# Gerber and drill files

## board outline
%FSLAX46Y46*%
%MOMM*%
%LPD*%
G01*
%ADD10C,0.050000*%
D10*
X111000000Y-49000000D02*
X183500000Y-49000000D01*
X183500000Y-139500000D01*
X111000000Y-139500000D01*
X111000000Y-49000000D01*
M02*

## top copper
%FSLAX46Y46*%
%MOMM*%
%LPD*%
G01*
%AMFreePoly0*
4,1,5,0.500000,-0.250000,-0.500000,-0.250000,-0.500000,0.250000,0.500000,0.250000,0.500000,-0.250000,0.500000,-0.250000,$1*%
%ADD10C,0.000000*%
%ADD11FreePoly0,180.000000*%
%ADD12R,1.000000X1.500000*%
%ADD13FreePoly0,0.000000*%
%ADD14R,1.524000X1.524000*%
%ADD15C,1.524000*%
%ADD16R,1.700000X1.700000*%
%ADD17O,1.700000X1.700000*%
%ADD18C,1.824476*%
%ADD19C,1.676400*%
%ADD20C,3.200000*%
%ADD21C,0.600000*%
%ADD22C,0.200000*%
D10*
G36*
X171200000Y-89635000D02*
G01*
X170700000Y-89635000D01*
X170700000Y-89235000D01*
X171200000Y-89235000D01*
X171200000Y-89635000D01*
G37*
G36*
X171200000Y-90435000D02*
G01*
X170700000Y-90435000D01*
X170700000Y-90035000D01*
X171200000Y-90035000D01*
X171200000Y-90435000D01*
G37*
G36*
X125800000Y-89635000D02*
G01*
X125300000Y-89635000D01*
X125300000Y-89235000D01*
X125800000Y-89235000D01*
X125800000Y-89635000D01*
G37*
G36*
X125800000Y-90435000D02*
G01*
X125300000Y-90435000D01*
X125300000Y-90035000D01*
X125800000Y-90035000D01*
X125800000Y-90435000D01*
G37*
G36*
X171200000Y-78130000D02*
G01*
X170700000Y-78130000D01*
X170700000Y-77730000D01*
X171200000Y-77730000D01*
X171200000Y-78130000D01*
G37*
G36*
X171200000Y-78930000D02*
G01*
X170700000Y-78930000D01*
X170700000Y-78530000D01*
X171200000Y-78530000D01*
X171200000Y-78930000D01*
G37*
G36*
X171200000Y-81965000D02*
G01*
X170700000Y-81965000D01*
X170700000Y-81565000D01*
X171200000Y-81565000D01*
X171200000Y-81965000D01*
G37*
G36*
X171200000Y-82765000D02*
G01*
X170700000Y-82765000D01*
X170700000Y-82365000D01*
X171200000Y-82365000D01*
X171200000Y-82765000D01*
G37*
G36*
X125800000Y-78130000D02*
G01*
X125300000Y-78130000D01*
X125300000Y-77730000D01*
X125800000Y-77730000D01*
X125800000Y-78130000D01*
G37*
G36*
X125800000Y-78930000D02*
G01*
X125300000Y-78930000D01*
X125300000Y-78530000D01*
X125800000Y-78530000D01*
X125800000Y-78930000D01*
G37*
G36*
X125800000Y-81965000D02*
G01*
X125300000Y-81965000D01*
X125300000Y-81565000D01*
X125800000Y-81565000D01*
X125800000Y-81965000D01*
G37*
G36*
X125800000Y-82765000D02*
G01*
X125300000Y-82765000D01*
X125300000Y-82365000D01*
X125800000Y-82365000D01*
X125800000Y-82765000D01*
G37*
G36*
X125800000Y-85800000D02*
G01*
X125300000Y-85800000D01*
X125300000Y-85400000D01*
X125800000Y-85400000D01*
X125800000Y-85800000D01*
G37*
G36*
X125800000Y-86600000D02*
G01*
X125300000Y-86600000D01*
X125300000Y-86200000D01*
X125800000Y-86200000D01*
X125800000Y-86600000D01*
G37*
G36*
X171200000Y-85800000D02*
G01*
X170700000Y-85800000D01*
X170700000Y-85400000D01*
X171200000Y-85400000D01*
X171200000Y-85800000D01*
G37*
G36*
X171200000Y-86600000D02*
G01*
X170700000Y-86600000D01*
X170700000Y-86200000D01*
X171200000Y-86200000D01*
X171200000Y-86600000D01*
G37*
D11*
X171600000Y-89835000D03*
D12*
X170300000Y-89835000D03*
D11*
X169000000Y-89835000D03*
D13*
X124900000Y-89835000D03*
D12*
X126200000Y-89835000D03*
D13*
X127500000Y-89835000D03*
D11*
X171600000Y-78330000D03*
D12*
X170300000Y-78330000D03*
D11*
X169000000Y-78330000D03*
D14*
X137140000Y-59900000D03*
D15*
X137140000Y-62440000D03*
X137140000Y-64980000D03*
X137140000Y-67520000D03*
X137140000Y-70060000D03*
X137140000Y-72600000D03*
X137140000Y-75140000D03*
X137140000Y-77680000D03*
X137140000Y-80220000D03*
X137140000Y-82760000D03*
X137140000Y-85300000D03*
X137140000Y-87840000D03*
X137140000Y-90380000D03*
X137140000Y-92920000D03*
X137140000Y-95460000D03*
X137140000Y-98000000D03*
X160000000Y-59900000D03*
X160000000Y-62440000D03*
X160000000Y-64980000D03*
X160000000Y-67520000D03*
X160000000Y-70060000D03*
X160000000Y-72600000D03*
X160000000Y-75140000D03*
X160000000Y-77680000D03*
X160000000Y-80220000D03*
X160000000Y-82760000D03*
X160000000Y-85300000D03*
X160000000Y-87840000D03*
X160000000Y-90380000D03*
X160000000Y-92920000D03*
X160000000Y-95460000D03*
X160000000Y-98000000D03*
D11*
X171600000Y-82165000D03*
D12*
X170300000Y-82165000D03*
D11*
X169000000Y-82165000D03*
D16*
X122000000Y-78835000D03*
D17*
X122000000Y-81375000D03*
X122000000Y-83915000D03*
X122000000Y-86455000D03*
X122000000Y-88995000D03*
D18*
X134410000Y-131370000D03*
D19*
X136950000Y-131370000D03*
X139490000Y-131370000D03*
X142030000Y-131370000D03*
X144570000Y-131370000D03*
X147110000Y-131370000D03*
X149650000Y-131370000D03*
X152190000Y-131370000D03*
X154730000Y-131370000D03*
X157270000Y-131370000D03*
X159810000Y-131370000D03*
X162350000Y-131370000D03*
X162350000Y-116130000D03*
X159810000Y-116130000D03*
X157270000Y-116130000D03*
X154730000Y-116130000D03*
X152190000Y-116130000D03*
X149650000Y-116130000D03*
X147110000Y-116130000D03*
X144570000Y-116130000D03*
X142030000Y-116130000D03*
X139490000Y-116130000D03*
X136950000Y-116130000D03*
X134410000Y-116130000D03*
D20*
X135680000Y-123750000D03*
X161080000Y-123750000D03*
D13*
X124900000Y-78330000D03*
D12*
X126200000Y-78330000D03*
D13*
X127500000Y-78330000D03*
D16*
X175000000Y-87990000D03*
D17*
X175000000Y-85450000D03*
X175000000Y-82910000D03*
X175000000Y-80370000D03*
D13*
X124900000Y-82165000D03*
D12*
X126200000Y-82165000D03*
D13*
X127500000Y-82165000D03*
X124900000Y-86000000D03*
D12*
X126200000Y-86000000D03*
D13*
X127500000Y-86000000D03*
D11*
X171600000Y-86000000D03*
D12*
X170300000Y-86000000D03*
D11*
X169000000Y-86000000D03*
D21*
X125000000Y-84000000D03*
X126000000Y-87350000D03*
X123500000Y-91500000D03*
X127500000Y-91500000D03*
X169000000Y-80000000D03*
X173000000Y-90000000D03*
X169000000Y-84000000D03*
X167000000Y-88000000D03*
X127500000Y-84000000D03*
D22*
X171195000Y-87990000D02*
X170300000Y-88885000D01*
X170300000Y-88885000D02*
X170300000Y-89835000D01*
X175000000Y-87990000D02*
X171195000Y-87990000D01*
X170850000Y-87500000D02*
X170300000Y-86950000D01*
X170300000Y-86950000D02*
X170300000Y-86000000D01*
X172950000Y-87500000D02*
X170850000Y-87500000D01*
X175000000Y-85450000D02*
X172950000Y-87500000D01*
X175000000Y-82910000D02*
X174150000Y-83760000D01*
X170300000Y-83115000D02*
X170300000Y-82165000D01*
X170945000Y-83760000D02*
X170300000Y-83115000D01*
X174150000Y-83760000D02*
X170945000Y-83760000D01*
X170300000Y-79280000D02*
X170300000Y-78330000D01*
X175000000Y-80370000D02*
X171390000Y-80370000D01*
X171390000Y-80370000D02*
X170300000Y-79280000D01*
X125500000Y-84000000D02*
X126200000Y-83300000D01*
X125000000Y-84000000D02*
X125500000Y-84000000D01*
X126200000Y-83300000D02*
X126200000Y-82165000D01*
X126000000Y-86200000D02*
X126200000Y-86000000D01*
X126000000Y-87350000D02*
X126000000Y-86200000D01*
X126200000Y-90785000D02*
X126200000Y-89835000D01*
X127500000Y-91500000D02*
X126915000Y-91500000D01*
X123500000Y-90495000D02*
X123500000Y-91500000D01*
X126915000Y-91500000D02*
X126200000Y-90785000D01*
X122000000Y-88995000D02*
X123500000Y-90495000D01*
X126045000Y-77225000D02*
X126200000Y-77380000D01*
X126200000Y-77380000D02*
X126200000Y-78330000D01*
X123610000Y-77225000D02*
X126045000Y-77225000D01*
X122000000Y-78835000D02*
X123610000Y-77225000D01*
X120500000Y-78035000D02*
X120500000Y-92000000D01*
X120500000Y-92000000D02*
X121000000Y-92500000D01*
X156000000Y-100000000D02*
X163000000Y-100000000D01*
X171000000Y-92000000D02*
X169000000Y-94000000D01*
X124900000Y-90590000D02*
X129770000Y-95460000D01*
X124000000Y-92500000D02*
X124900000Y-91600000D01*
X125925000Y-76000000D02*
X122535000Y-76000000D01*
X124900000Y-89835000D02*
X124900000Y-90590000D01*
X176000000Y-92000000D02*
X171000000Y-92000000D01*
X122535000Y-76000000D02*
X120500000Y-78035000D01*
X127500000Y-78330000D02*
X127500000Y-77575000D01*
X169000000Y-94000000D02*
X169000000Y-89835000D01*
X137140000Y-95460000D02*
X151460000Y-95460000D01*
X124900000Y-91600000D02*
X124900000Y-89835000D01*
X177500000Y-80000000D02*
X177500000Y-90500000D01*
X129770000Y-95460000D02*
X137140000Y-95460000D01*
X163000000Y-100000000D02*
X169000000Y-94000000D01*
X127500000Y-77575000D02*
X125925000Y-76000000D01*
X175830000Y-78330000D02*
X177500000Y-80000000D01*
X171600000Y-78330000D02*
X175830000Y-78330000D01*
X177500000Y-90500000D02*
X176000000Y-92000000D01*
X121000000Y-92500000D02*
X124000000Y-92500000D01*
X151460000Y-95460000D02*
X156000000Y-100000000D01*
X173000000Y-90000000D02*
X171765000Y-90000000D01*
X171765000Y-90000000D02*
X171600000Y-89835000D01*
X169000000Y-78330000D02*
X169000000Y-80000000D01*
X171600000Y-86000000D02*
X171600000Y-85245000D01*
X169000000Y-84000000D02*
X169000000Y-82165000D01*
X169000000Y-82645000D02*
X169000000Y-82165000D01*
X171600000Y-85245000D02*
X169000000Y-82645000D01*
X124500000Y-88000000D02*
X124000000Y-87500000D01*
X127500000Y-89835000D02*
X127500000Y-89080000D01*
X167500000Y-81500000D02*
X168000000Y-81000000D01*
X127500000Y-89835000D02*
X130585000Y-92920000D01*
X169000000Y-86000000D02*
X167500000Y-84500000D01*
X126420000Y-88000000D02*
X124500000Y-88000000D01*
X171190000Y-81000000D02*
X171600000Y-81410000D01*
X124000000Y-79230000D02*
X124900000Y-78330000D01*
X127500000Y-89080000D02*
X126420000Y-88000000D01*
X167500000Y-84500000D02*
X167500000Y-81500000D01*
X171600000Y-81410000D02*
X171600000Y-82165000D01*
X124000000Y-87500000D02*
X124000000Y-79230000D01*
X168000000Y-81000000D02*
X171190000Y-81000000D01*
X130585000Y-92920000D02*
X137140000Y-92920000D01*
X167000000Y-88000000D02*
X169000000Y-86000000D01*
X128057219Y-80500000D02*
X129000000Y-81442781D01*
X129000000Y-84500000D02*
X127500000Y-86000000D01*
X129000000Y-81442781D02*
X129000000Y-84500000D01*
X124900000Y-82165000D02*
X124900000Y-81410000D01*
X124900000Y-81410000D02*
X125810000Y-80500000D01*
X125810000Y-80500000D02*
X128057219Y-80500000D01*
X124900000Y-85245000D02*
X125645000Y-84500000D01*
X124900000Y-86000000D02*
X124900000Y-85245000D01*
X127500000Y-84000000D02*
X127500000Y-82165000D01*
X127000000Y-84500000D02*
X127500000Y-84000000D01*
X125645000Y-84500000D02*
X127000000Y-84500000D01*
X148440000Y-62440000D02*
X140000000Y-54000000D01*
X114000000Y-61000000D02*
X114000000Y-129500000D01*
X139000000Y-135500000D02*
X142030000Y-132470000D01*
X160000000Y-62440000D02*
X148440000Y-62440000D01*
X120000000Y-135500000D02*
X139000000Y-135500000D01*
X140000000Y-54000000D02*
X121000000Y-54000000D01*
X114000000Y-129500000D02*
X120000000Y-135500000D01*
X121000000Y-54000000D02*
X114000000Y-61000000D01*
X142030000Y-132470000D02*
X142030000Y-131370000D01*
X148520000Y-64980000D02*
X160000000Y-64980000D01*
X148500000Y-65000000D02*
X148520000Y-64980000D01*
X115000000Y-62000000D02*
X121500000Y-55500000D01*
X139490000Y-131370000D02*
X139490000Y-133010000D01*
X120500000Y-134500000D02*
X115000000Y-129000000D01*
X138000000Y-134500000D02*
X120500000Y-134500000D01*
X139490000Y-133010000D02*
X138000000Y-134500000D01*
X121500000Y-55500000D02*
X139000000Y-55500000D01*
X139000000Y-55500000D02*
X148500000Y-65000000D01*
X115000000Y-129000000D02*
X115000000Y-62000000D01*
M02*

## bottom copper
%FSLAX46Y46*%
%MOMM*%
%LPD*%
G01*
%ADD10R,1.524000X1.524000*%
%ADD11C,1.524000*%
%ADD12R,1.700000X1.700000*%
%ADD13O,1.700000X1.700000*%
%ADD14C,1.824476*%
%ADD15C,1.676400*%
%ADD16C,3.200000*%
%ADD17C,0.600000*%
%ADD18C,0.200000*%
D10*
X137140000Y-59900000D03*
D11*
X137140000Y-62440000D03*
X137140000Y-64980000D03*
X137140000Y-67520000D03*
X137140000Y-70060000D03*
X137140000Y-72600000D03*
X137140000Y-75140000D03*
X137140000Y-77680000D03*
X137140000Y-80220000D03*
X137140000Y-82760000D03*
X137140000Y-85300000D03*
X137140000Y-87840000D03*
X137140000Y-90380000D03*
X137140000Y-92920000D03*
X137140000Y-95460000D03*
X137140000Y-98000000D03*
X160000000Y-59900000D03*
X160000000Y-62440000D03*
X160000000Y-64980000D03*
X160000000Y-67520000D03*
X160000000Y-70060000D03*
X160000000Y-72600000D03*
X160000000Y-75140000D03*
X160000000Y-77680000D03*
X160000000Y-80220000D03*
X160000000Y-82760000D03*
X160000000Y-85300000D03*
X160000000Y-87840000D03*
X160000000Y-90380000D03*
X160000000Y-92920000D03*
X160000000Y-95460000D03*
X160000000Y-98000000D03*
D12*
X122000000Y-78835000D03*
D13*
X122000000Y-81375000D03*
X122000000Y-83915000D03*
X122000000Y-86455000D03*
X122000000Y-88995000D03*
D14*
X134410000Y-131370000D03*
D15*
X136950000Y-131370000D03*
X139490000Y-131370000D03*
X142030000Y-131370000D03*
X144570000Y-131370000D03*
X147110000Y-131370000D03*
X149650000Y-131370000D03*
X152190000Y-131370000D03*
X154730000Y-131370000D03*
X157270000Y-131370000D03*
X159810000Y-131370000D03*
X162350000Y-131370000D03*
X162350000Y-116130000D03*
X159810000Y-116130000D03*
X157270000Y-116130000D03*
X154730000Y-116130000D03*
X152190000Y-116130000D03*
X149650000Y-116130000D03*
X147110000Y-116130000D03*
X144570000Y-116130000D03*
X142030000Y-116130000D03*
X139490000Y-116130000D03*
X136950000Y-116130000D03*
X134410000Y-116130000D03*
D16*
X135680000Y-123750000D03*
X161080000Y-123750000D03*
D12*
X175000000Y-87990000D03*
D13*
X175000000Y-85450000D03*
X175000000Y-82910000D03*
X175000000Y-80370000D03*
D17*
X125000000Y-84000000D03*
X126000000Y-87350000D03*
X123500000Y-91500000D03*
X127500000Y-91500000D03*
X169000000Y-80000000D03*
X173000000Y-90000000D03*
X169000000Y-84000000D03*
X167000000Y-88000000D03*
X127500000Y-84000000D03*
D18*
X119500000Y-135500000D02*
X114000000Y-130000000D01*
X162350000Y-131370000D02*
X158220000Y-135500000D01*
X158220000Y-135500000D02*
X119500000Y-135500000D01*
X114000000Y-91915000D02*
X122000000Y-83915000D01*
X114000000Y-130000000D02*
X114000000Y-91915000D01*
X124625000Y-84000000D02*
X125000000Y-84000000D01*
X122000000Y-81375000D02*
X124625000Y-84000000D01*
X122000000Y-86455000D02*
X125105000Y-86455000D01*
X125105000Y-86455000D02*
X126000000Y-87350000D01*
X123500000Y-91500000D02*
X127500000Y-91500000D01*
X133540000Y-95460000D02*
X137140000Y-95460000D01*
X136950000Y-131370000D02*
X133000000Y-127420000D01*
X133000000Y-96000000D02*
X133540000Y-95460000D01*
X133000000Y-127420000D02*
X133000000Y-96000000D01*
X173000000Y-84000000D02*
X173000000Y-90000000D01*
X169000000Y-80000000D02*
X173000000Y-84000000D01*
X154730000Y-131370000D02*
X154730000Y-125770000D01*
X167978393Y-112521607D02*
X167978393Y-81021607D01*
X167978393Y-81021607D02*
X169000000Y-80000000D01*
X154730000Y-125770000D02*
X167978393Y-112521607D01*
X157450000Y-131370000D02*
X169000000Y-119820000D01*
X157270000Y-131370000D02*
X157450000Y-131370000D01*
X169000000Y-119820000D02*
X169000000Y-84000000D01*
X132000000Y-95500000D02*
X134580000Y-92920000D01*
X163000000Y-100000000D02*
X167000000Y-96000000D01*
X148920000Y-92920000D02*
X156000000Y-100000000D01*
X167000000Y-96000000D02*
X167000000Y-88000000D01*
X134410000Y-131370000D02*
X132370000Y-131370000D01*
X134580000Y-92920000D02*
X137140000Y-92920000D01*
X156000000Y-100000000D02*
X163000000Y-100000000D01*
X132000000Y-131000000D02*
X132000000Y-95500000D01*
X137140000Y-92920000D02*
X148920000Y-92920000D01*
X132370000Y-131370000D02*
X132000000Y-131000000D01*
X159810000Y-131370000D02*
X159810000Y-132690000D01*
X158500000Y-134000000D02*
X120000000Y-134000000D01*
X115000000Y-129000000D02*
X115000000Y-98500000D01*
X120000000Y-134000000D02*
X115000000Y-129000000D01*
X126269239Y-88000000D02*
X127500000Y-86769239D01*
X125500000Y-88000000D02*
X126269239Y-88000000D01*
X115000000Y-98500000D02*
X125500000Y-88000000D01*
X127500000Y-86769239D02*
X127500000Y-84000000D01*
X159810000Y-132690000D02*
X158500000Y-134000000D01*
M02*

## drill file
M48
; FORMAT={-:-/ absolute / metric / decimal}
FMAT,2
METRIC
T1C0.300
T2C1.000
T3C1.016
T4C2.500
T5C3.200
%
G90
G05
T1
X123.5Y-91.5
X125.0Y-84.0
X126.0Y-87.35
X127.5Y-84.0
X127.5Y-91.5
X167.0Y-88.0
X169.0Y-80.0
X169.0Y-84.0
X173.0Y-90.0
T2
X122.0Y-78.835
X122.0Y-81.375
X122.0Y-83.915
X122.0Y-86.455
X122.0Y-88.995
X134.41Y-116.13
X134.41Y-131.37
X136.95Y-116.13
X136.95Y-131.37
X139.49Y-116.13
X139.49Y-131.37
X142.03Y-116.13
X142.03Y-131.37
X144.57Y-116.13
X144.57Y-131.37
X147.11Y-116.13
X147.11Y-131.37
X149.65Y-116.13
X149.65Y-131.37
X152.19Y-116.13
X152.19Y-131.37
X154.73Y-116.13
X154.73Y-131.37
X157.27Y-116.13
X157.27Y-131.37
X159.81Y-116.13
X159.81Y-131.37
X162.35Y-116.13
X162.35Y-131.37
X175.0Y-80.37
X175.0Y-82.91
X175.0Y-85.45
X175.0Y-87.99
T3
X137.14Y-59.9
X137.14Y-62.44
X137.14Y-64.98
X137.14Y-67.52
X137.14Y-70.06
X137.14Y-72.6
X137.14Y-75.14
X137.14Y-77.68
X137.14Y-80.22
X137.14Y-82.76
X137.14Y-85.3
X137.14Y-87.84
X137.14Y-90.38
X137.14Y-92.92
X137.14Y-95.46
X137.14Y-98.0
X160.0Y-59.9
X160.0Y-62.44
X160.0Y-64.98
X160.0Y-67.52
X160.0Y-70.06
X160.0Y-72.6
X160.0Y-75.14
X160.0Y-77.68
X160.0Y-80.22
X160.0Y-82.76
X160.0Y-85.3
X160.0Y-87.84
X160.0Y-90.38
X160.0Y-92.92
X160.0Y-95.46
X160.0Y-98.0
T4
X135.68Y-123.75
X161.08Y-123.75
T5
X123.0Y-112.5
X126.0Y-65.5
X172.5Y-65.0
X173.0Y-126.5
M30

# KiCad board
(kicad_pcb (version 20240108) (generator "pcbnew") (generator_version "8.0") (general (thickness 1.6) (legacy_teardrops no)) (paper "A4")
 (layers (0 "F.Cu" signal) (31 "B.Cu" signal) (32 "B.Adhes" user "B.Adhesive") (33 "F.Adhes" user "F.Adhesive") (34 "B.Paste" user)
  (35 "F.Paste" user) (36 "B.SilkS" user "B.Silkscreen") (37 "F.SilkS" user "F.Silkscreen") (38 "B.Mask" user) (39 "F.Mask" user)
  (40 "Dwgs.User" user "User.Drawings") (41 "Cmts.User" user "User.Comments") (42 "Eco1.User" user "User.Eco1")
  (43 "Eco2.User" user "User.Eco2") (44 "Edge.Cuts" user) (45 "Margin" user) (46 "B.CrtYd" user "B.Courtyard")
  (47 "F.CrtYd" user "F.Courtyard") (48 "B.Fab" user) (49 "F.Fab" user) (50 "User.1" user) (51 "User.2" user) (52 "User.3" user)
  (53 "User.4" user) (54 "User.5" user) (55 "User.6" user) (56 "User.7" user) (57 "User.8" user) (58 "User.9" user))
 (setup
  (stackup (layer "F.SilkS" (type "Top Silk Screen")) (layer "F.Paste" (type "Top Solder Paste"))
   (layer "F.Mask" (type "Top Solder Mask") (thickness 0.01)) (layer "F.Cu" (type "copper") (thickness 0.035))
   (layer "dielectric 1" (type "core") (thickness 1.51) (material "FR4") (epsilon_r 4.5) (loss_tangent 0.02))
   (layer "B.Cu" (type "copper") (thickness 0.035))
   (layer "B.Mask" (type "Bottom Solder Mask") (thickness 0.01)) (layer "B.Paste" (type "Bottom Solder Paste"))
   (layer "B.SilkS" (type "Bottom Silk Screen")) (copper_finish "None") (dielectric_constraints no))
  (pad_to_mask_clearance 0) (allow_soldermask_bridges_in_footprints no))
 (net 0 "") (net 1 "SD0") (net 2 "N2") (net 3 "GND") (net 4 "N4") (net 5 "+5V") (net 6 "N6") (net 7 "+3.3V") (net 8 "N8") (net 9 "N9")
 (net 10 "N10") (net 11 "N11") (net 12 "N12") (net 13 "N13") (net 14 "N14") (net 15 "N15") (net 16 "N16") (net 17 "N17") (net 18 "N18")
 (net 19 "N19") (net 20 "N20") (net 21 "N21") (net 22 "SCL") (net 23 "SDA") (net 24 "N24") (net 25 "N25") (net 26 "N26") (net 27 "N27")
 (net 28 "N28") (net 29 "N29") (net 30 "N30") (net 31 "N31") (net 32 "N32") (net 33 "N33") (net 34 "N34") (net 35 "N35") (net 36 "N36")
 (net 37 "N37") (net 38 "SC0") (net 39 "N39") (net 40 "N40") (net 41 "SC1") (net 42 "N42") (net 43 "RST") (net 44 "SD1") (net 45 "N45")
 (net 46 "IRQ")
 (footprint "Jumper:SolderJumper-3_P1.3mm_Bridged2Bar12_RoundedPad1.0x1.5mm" (layer "F.Cu") (at 170.3 89.835 180)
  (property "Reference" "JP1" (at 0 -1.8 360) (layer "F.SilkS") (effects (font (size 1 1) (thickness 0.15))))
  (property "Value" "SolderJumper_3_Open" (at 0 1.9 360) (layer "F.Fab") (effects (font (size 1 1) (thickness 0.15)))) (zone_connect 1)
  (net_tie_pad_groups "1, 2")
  (fp_poly (pts (xy -0.9 0.2) (xy -0.4 0.2) (xy -0.4 0.6) (xy -0.9 0.6)) (stroke (width 0) (type solid)) (fill solid) (layer "F.Cu"))
  (fp_poly (pts (xy -0.9 -0.6) (xy -0.4 -0.6) (xy -0.4 -0.2) (xy -0.9 -0.2)) (stroke (width 0) (type solid)) (fill solid) (layer "F.Cu"))
  (pad "1" smd custom (at -1.3 0 180) (size 1 0.5) (layers "F.Cu" "F.Mask") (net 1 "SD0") (zone_connect 2) (thermal_bridge_angle 45)
   (options (clearance outline) (anchor rect)) (primitives))
  (pad "2" smd rect (at 0 0 180) (size 1 1.5) (layers "F.Cu" "F.Mask") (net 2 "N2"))
  (pad "3" smd custom (at 1.3 0 180) (size 1 0.5) (layers "F.Cu" "F.Mask") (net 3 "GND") (zone_connect 2) (thermal_bridge_angle 45)
   (options (clearance outline) (anchor rect)) (primitives)))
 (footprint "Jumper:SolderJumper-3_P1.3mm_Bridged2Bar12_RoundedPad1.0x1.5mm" (layer "F.Cu") (at 126.2 89.835)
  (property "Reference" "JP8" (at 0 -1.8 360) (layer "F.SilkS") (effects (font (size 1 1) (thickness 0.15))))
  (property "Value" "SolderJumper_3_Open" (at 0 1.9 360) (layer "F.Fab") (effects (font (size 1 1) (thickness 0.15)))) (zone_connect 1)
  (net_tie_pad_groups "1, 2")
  (fp_poly (pts (xy -0.9 -0.6) (xy -0.4 -0.6) (xy -0.4 -0.2) (xy -0.9 -0.2)) (stroke (width 0) (type solid)) (fill solid) (layer "F.Cu"))
  (fp_poly (pts (xy -0.9 0.2) (xy -0.4 0.2) (xy -0.4 0.6) (xy -0.9 0.6)) (stroke (width 0) (type solid)) (fill solid) (layer "F.Cu"))
  (pad "1" smd custom (at -1.3 0) (size 1 0.5) (layers "F.Cu" "F.Mask") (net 3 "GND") (zone_connect 2) (thermal_bridge_angle 45)
   (options (clearance outline) (anchor rect)) (primitives))
  (pad "2" smd rect (at 0 0) (size 1 1.5) (layers "F.Cu" "F.Mask") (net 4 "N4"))
  (pad "3" smd custom (at 1.3 0) (size 1 0.5) (layers "F.Cu" "F.Mask") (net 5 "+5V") (zone_connect 2) (thermal_bridge_angle 45)
   (options (clearance outline) (anchor rect)) (primitives)))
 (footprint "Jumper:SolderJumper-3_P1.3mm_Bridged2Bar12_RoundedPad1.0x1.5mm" (layer "F.Cu") (at 170.3 78.33 180)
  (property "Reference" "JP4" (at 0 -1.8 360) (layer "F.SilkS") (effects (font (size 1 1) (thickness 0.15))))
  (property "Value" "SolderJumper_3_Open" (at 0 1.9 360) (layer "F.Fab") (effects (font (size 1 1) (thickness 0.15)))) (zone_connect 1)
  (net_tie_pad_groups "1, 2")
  (fp_poly (pts (xy -0.9 0.2) (xy -0.4 0.2) (xy -0.4 0.6) (xy -0.9 0.6)) (stroke (width 0) (type solid)) (fill solid) (layer "F.Cu"))
  (fp_poly (pts (xy -0.9 -0.6) (xy -0.4 -0.6) (xy -0.4 -0.2) (xy -0.9 -0.2)) (stroke (width 0) (type solid)) (fill solid) (layer "F.Cu"))
  (pad "1" smd custom (at -1.3 0 180) (size 1 0.5) (layers "F.Cu" "F.Mask") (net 3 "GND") (zone_connect 2) (thermal_bridge_angle 45)
   (options (clearance outline) (anchor rect)) (primitives))
  (pad "2" smd rect (at 0 0 180) (size 1 1.5) (layers "F.Cu" "F.Mask") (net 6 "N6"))
  (pad "3" smd custom (at 1.3 0 180) (size 1 0.5) (layers "F.Cu" "F.Mask") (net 1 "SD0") (zone_connect 2) (thermal_bridge_angle 45)
   (options (clearance outline) (anchor rect)) (primitives)))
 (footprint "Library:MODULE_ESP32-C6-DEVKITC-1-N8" (layer "F.Cu") (at 148.57 84.225)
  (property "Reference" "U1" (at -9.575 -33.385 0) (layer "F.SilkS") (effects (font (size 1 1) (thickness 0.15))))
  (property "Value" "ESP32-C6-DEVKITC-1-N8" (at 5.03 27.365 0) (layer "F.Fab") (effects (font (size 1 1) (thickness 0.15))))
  (pad "J1_1" thru_hole rect (at -11.43 -24.325) (size 1.524 1.524) (drill 1.016) (layers "*.Cu" "*.Mask") (remove_unused_layers no)
   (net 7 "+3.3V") (solder_mask_margin 0.102))
  (pad "J1_2" thru_hole circle (at -11.43 -21.785) (size 1.524 1.524) (drill 1.016) (layers "*.Cu" "*.Mask") (remove_unused_layers no)
   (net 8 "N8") (solder_mask_margin 0.102))
  (pad "J1_3" thru_hole circle (at -11.43 -19.245) (size 1.524 1.524) (drill 1.016) (layers "*.Cu" "*.Mask") (remove_unused_layers no)
   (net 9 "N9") (solder_mask_margin 0.102))
  (pad "J1_4" thru_hole circle (at -11.43 -16.705) (size 1.524 1.524) (drill 1.016) (layers "*.Cu" "*.Mask") (remove_unused_layers no)
   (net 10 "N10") (solder_mask_margin 0.102))
  (pad "J1_5" thru_hole circle (at -11.43 -14.165) (size 1.524 1.524) (drill 1.016) (layers "*.Cu" "*.Mask") (remove_unused_layers no)
   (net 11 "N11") (solder_mask_margin 0.102))
  (pad "J1_6" thru_hole circle (at -11.43 -11.625) (size 1.524 1.524) (drill 1.016) (layers "*.Cu" "*.Mask") (remove_unused_layers no)
   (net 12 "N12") (solder_mask_margin 0.102))
  (pad "J1_7" thru_hole circle (at -11.43 -9.085) (size 1.524 1.524) (drill 1.016) (layers "*.Cu" "*.Mask") (remove_unused_layers no)
   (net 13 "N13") (solder_mask_margin 0.102))
  (pad "J1_8" thru_hole circle (at -11.43 -6.545) (size 1.524 1.524) (drill 1.016) (layers "*.Cu" "*.Mask") (remove_unused_layers no)
   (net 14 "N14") (solder_mask_margin 0.102))
  (pad "J1_9" thru_hole circle (at -11.43 -4.005) (size 1.524 1.524) (drill 1.016) (layers "*.Cu" "*.Mask") (remove_unused_layers no)
   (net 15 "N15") (solder_mask_margin 0.102))
  (pad "J1_10" thru_hole circle (at -11.43 -1.465) (size 1.524 1.524) (drill 1.016) (layers "*.Cu" "*.Mask") (remove_unused_layers no)
   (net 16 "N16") (solder_mask_margin 0.102))
  (pad "J1_11" thru_hole circle (at -11.43 1.075) (size 1.524 1.524) (drill 1.016) (layers "*.Cu" "*.Mask") (remove_unused_layers no)
   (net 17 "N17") (solder_mask_margin 0.102))
  (pad "J1_12" thru_hole circle (at -11.43 3.615) (size 1.524 1.524) (drill 1.016) (layers "*.Cu" "*.Mask") (remove_unused_layers no)
   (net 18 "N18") (solder_mask_margin 0.102))
  (pad "J1_13" thru_hole circle (at -11.43 6.155) (size 1.524 1.524) (drill 1.016) (layers "*.Cu" "*.Mask") (remove_unused_layers no)
   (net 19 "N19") (solder_mask_margin 0.102))
  (pad "J1_14" thru_hole circle (at -11.43 8.695) (size 1.524 1.524) (drill 1.016) (layers "*.Cu" "*.Mask") (remove_unused_layers no)
   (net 5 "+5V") (solder_mask_margin 0.102))
  (pad "J1_15" thru_hole circle (at -11.43 11.235) (size 1.524 1.524) (drill 1.016) (layers "*.Cu" "*.Mask") (remove_unused_layers no)
   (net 3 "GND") (solder_mask_margin 0.102))
  (pad "J1_16" thru_hole circle (at -11.43 13.775) (size 1.524 1.524) (drill 1.016) (layers "*.Cu" "*.Mask") (remove_unused_layers no)
   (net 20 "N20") (solder_mask_margin 0.102))
  (pad "J3_1" thru_hole circle (at 11.43 -24.325) (size 1.524 1.524) (drill 1.016) (layers "*.Cu" "*.Mask") (remove_unused_layers no)
   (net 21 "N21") (solder_mask_margin 0.102))
  (pad "J3_2" thru_hole circle (at 11.43 -21.785) (size 1.524 1.524) (drill 1.016) (layers "*.Cu" "*.Mask") (remove_unused_layers no)
   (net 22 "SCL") (solder_mask_margin 0.102))
  (pad "J3_3" thru_hole circle (at 11.43 -19.245) (size 1.524 1.524) (drill 1.016) (layers "*.Cu" "*.Mask") (remove_unused_layers no)
   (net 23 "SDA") (solder_mask_margin 0.102))
  (pad "J3_4" thru_hole circle (at 11.43 -16.705) (size 1.524 1.524) (drill 1.016) (layers "*.Cu" "*.Mask") (remove_unused_layers no)
   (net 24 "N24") (solder_mask_margin 0.102))
  (pad "J3_5" thru_hole circle (at 11.43 -14.165) (size 1.524 1.524) (drill 1.016) (layers "*.Cu" "*.Mask") (remove_unused_layers no)
   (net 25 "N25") (solder_mask_margin 0.102))
  (pad "J3_6" thru_hole circle (at 11.43 -11.625) (size 1.524 1.524) (drill 1.016) (layers "*.Cu" "*.Mask") (remove_unused_layers no)
   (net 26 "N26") (solder_mask_margin 0.102))
  (pad "J3_7" thru_hole circle (at 11.43 -9.085) (size 1.524 1.524) (drill 1.016) (layers "*.Cu" "*.Mask") (remove_unused_layers no)
   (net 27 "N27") (solder_mask_margin 0.102))
  (pad "J3_8" thru_hole circle (at 11.43 -6.545) (size 1.524 1.524) (drill 1.016) (layers "*.Cu" "*.Mask") (remove_unused_layers no)
   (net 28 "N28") (solder_mask_margin 0.102))
  (pad "J3_9" thru_hole circle (at 11.43 -4.005) (size 1.524 1.524) (drill 1.016) (layers "*.Cu" "*.Mask") (remove_unused_layers no)
   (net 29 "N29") (solder_mask_margin 0.102))
  (pad "J3_10" thru_hole circle (at 11.43 -1.465) (size 1.524 1.524) (drill 1.016) (layers "*.Cu" "*.Mask") (remove_unused_layers no)
   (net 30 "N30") (solder_mask_margin 0.102))
  (pad "J3_11" thru_hole circle (at 11.43 1.075) (size 1.524 1.524) (drill 1.016) (layers "*.Cu" "*.Mask") (remove_unused_layers no)
   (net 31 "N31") (solder_mask_margin 0.102))
  (pad "J3_12" thru_hole circle (at 11.43 3.615) (size 1.524 1.524) (drill 1.016) (layers "*.Cu" "*.Mask") (remove_unused_layers no)
   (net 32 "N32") (solder_mask_margin 0.102))
  (pad "J3_13" thru_hole circle (at 11.43 6.155) (size 1.524 1.524) (drill 1.016) (layers "*.Cu" "*.Mask") (remove_unused_layers no)
   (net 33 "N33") (solder_mask_margin 0.102))
  (pad "J3_14" thru_hole circle (at 11.43 8.695) (size 1.524 1.524) (drill 1.016) (layers "*.Cu" "*.Mask") (remove_unused_layers no)
   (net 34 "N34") (solder_mask_margin 0.102))
  (pad "J3_15" thru_hole circle (at 11.43 11.235) (size 1.524 1.524) (drill 1.016) (layers "*.Cu" "*.Mask") (remove_unused_layers no)
   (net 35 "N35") (solder_mask_margin 0.102))
  (pad "J3_16" thru_hole circle (at 11.43 13.775) (size 1.524 1.524) (drill 1.016) (layers "*.Cu" "*.Mask") (remove_unused_layers no)
   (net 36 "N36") (solder_mask_margin 0.102)))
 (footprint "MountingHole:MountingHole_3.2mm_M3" (layer "F.Cu") (at 173 126.5)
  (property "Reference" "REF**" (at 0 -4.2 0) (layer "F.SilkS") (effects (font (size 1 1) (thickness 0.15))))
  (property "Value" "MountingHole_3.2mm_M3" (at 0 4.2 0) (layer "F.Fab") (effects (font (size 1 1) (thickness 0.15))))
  (pad "" np_thru_hole circle (at 0 0) (size 3.2 3.2) (drill 3.2) (layers "F&B.Cu" "*.Mask")))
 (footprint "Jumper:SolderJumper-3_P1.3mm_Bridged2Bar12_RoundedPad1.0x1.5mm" (layer "F.Cu") (at 170.3 82.165 180)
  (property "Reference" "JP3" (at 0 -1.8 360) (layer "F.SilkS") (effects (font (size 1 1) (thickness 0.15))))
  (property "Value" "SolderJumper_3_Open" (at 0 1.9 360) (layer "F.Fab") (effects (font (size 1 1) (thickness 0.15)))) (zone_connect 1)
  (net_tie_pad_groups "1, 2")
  (fp_poly (pts (xy -0.9 0.2) (xy -0.4 0.2) (xy -0.4 0.6) (xy -0.9 0.6)) (stroke (width 0) (type solid)) (fill solid) (layer "F.Cu"))
  (fp_poly (pts (xy -0.9 -0.6) (xy -0.4 -0.6) (xy -0.4 -0.2) (xy -0.9 -0.2)) (stroke (width 0) (type solid)) (fill solid) (layer "F.Cu"))
  (pad "1" smd custom (at -1.3 0 180) (size 1 0.5) (layers "F.Cu" "F.Mask") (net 5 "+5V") (zone_connect 2) (thermal_bridge_angle 45)
   (options (clearance outline) (anchor rect)) (primitives))
  (pad "2" smd rect (at 0 0 180) (size 1 1.5) (layers "F.Cu" "F.Mask") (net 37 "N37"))
  (pad "3" smd custom (at 1.3 0 180) (size 1 0.5) (layers "F.Cu" "F.Mask") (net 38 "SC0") (zone_connect 2) (thermal_bridge_angle 45)
   (options (clearance outline) (anchor rect)) (primitives)))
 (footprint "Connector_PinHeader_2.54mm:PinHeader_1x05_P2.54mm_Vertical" (layer "F.Cu") (at 122 78.835)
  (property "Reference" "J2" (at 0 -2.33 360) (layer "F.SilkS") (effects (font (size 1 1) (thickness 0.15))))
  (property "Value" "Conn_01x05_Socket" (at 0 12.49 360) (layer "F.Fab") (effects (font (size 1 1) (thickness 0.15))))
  (pad "1" thru_hole rect (at 0 0) (size 1.7 1.7) (drill 1) (layers "*.Cu" "*.Mask") (remove_unused_layers no) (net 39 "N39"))
  (pad "2" thru_hole oval (at 0 2.54) (size 1.7 1.7) (drill 1) (layers "*.Cu" "*.Mask") (remove_unused_layers no) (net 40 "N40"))
  (pad "3" thru_hole oval (at 0 5.08) (size 1.7 1.7) (drill 1) (layers "*.Cu" "*.Mask") (remove_unused_layers no) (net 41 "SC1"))
  (pad "4" thru_hole oval (at 0 7.62) (size 1.7 1.7) (drill 1) (layers "*.Cu" "*.Mask") (remove_unused_layers no) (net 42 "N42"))
  (pad "5" thru_hole oval (at 0 10.16) (size 1.7 1.7) (drill 1) (layers "*.Cu" "*.Mask") (remove_unused_layers no) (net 4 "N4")))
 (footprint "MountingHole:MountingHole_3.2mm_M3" (layer "F.Cu") (at 123 112.5)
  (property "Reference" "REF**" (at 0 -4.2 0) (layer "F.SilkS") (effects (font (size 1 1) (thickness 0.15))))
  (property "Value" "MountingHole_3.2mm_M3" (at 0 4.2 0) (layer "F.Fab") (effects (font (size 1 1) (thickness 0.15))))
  (pad "" np_thru_hole circle (at 0 0) (size 3.2 3.2) (drill 3.2) (layers "F&B.Cu" "*.Mask")))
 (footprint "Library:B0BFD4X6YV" (layer "F.Cu") (at 129.27 123.13 90)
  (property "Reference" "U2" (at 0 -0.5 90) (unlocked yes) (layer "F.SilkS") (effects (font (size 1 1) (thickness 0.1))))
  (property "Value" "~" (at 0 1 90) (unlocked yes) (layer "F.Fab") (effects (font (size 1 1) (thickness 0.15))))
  (pad "1" thru_hole circle (at -8.24 5.14 90) (size 1.824476 1.824476) (drill 1) (layers "*.Cu" "*.Mask") (remove_unused_layers no)
   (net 5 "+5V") (solder_mask_margin 0.0508) (thermal_bridge_angle 0))
  (pad "2" thru_hole circle (at -8.24 7.68 90) (size 1.6764 1.6764) (drill 1) (layers "*.Cu" "*.Mask") (remove_unused_layers no)
   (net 3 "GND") (solder_mask_margin 0.0508) (thermal_bridge_angle 0))
  (pad "3" thru_hole circle (at -8.24 10.22 90) (size 1.6764 1.6764) (drill 1) (layers "*.Cu" "*.Mask") (remove_unused_layers no)
   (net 23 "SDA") (solder_mask_margin 0.0508) (thermal_bridge_angle 0))
  (pad "4" thru_hole circle (at -8.24 12.76 90) (size 1.6764 1.6764) (drill 1) (layers "*.Cu" "*.Mask") (remove_unused_layers no)
   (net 22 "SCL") (solder_mask_margin 0.0508) (thermal_bridge_angle 0))
  (pad "5" thru_hole circle (at -8.24 15.3 90) (size 1.6764 1.6764) (drill 1) (layers "*.Cu" "*.Mask") (remove_unused_layers no)
   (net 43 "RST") (solder_mask_margin 0.0508) (thermal_bridge_angle 0))
  (pad "6" thru_hole circle (at -8.24 17.84 90) (size 1.6764 1.6764) (drill 1) (layers "*.Cu" "*.Mask") (remove_unused_layers no)
   (solder_mask_margin 0.0508) (thermal_bridge_angle 0))
  (pad "7" thru_hole circle (at -8.24 20.38 90) (size 1.6764 1.6764) (drill 1) (layers "*.Cu" "*.Mask") (remove_unused_layers no)
   (solder_mask_margin 0.0508) (thermal_bridge_angle 0))
  (pad "8" thru_hole circle (at -8.24 22.92 90) (size 1.6764 1.6764) (drill 1) (layers "*.Cu" "*.Mask") (remove_unused_layers no)
   (solder_mask_margin 0.0508) (thermal_bridge_angle 0))
  (pad "9" thru_hole circle (at -8.24 25.46 90) (size 1.6764 1.6764) (drill 1) (layers "*.Cu" "*.Mask") (remove_unused_layers no)
   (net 1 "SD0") (solder_mask_margin 0.0508) (thermal_bridge_angle 0))
  (pad "10" thru_hole circle (at -8.24 28 90) (size 1.6764 1.6764) (drill 1) (layers "*.Cu" "*.Mask") (remove_unused_layers no)
   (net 38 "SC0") (solder_mask_margin 0.0508) (thermal_bridge_angle 0))
  (pad "11" thru_hole circle (at -8.24 30.54 90) (size 1.6764 1.6764) (drill 1) (layers "*.Cu" "*.Mask") (remove_unused_layers no)
   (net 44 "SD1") (solder_mask_margin 0.0508) (thermal_bridge_angle 0))
  (pad "12" thru_hole circle (at -8.24 33.08 90) (size 1.6764 1.6764) (drill 1) (layers "*.Cu" "*.Mask") (remove_unused_layers no)
   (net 41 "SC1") (solder_mask_margin 0.0508) (thermal_bridge_angle 0))
  (pad "13" thru_hole circle (at 7 33.08 270) (size 1.6764 1.6764) (drill 1) (layers "*.Cu" "*.Mask") (remove_unused_layers no)
   (solder_mask_margin 0.0508) (thermal_bridge_angle 0))
  (pad "14" thru_hole circle (at 7 30.54 270) (size 1.6764 1.6764) (drill 1) (layers "*.Cu" "*.Mask") (remove_unused_layers no)
   (solder_mask_margin 0.0508) (thermal_bridge_angle 0))
  (pad "15" thru_hole circle (at 7 28 270) (size 1.6764 1.6764) (drill 1) (layers "*.Cu" "*.Mask") (remove_unused_layers no)
   (solder_mask_margin 0.0508) (thermal_bridge_angle 0))
  (pad "16" thru_hole circle (at 7 25.46 270) (size 1.6764 1.6764) (drill 1) (layers "*.Cu" "*.Mask") (remove_unused_layers no)
   (solder_mask_margin 0.0508) (thermal_bridge_angle 0))
  (pad "17" thru_hole circle (at 7 22.92 270) (size 1.6764 1.6764) (drill 1) (layers "*.Cu" "*.Mask") (remove_unused_layers no)
   (solder_mask_margin 0.0508) (thermal_bridge_angle 0))
  (pad "18" thru_hole circle (at 7 20.38 270) (size 1.6764 1.6764) (drill 1) (layers "*.Cu" "*.Mask") (remove_unused_layers no)
   (solder_mask_margin 0.0508) (thermal_bridge_angle 0))
  (pad "19" thru_hole circle (at 7 17.84 270) (size 1.6764 1.6764) (drill 1) (layers "*.Cu" "*.Mask") (remove_unused_layers no)
   (solder_mask_margin 0.0508) (thermal_bridge_angle 0))
  (pad "20" thru_hole circle (at 7 15.3 270) (size 1.6764 1.6764) (drill 1) (layers "*.Cu" "*.Mask") (remove_unused_layers no)
   (solder_mask_margin 0.0508) (thermal_bridge_angle 0))
  (pad "21" thru_hole circle (at 7 12.76 270) (size 1.6764 1.6764) (drill 1) (layers "*.Cu" "*.Mask") (remove_unused_layers no)
   (solder_mask_margin 0.0508) (thermal_bridge_angle 0))
  (pad "22" thru_hole circle (at 7 10.22 270) (size 1.6764 1.6764) (drill 1) (layers "*.Cu" "*.Mask") (remove_unused_layers no)
   (solder_mask_margin 0.0508) (thermal_bridge_angle 0))
  (pad "23" thru_hole circle (at 7 7.68 270) (size 1.6764 1.6764) (drill 1) (layers "*.Cu" "*.Mask") (remove_unused_layers no)
   (solder_mask_margin 0.0508) (thermal_bridge_angle 0))
  (pad "24" thru_hole circle (at 7 5.14 270) (size 1.6764 1.6764) (drill 1) (layers "*.Cu" "*.Mask") (remove_unused_layers no)
   (solder_mask_margin 0.0508) (thermal_bridge_angle 0))
  (pad "P$1" thru_hole circle (at -0.62 6.41 90) (size 3.2 3.2) (drill 2.5) (layers "*.Cu" "*.Mask") (remove_unused_layers no)
   (solder_mask_margin 0.0508) (thermal_bridge_angle 0))
  (pad "P$1" thru_hole circle (at -0.62 31.81 90) (size 3.2 3.2) (drill 2.5) (layers "*.Cu" "*.Mask") (remove_unused_layers no)
   (solder_mask_margin 0.0508) (thermal_bridge_angle 0)))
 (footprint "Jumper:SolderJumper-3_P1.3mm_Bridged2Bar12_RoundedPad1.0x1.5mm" (layer "F.Cu") (at 126.2 78.33)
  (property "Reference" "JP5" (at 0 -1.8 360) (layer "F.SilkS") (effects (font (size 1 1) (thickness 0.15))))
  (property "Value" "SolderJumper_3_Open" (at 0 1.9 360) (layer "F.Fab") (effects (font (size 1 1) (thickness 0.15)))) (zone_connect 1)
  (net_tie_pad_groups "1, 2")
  (fp_poly (pts (xy -0.9 -0.6) (xy -0.4 -0.6) (xy -0.4 -0.2) (xy -0.9 -0.2)) (stroke (width 0) (type solid)) (fill solid) (layer "F.Cu"))
  (fp_poly (pts (xy -0.9 0.2) (xy -0.4 0.2) (xy -0.4 0.6) (xy -0.9 0.6)) (stroke (width 0) (type solid)) (fill solid) (layer "F.Cu"))
  (pad "1" smd custom (at -1.3 0) (size 1 0.5) (layers "F.Cu" "F.Mask") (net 5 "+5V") (zone_connect 2) (thermal_bridge_angle 45)
   (options (clearance outline) (anchor rect)) (primitives))
  (pad "2" smd rect (at 0 0) (size 1 1.5) (layers "F.Cu" "F.Mask") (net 39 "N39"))
  (pad "3" smd custom (at 1.3 0) (size 1 0.5) (layers "F.Cu" "F.Mask") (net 3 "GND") (zone_connect 2) (thermal_bridge_angle 45)
   (options (clearance outline) (anchor rect)) (primitives)))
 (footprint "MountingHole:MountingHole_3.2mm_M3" (layer "F.Cu") (at 172.5 65)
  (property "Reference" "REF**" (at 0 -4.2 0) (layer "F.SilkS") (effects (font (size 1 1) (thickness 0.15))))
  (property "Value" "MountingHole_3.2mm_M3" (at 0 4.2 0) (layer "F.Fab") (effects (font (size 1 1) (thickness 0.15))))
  (pad "" np_thru_hole circle (at 0 0) (size 3.2 3.2) (drill 3.2) (layers "F&B.Cu" "*.Mask")))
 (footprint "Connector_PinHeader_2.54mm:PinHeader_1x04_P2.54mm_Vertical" (layer "F.Cu") (at 175 87.99 180)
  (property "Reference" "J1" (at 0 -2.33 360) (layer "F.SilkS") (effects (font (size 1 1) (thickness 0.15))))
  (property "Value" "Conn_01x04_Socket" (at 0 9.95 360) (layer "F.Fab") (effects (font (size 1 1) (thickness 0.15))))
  (pad "1" thru_hole rect (at 0 0 180) (size 1.7 1.7) (drill 1) (layers "*.Cu" "*.Mask") (remove_unused_layers no) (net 2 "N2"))
  (pad "2" thru_hole oval (at 0 2.54 180) (size 1.7 1.7) (drill 1) (layers "*.Cu" "*.Mask") (remove_unused_layers no) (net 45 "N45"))
  (pad "3" thru_hole oval (at 0 5.08 180) (size 1.7 1.7) (drill 1) (layers "*.Cu" "*.Mask") (remove_unused_layers no) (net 37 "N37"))
  (pad "4" thru_hole oval (at 0 7.62 180) (size 1.7 1.7) (drill 1) (layers "*.Cu" "*.Mask") (remove_unused_layers no) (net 6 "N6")))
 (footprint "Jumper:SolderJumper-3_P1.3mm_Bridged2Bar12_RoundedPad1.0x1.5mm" (layer "F.Cu") (at 126.2 82.165)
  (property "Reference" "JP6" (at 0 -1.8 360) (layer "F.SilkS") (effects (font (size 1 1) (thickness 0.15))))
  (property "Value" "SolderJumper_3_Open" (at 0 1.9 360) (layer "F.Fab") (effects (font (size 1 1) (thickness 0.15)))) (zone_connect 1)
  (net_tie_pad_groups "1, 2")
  (fp_poly (pts (xy -0.9 -0.6) (xy -0.4 -0.6) (xy -0.4 -0.2) (xy -0.9 -0.2)) (stroke (width 0) (type solid)) (fill solid) (layer "F.Cu"))
  (fp_poly (pts (xy -0.9 0.2) (xy -0.4 0.2) (xy -0.4 0.6) (xy -0.9 0.6)) (stroke (width 0) (type solid)) (fill solid) (layer "F.Cu"))
  (pad "1" smd custom (at -1.3 0) (size 1 0.5) (layers "F.Cu" "F.Mask") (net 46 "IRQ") (zone_connect 2) (thermal_bridge_angle 45)
   (options (clearance outline) (anchor rect)) (primitives))
  (pad "2" smd rect (at 0 0) (size 1 1.5) (layers "F.Cu" "F.Mask") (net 40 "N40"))
  (pad "3" smd custom (at 1.3 0) (size 1 0.5) (layers "F.Cu" "F.Mask") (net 44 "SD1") (zone_connect 2) (thermal_bridge_angle 45)
   (options (clearance outline) (anchor rect)) (primitives)))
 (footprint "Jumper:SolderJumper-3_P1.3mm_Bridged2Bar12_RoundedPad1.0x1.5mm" (layer "F.Cu") (at 126.2 86)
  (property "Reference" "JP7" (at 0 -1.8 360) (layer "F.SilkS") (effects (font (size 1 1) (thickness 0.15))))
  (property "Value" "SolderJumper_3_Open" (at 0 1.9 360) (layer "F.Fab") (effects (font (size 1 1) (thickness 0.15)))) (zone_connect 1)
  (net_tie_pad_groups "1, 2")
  (fp_poly (pts (xy -0.9 -0.6) (xy -0.4 -0.6) (xy -0.4 -0.2) (xy -0.9 -0.2)) (stroke (width 0) (type solid)) (fill solid) (layer "F.Cu"))
  (fp_poly (pts (xy -0.9 0.2) (xy -0.4 0.2) (xy -0.4 0.6) (xy -0.9 0.6)) (stroke (width 0) (type solid)) (fill solid) (layer "F.Cu"))
  (pad "1" smd custom (at -1.3 0) (size 1 0.5) (layers "F.Cu" "F.Mask") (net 44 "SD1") (zone_connect 2) (thermal_bridge_angle 45)
   (options (clearance outline) (anchor rect)) (primitives))
  (pad "2" smd rect (at 0 0) (size 1 1.5) (layers "F.Cu" "F.Mask") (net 42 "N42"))
  (pad "3" smd custom (at 1.3 0) (size 1 0.5) (layers "F.Cu" "F.Mask") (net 46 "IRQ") (zone_connect 2) (thermal_bridge_angle 45)
   (options (clearance outline) (anchor rect)) (primitives)))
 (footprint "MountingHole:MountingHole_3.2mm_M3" (layer "F.Cu") (at 126 65.5)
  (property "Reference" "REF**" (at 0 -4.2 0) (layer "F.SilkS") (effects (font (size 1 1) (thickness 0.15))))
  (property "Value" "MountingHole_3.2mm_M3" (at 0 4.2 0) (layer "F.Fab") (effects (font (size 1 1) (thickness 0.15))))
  (pad "" np_thru_hole circle (at 0 0) (size 3.2 3.2) (drill 3.2) (layers "*.Cu" "*.Mask")))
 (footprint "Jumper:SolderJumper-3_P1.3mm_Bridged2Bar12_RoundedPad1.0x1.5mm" (layer "F.Cu") (at 170.3 86 180)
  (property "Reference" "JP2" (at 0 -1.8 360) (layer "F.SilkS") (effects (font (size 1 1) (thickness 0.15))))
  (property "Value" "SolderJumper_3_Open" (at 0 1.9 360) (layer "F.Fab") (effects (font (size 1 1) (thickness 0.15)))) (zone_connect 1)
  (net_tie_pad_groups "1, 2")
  (fp_poly (pts (xy -0.9 0.2) (xy -0.4 0.2) (xy -0.4 0.6) (xy -0.9 0.6)) (stroke (width 0) (type solid)) (fill solid) (layer "F.Cu"))
  (fp_poly (pts (xy -0.9 -0.6) (xy -0.4 -0.6) (xy -0.4 -0.2) (xy -0.9 -0.2)) (stroke (width 0) (type solid)) (fill solid) (layer "F.Cu"))
  (pad "1" smd custom (at -1.3 0 180) (size 1 0.5) (layers "F.Cu" "F.Mask") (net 38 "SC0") (zone_connect 2) (thermal_bridge_angle 45)
   (options (clearance outline) (anchor rect)) (primitives))
  (pad "2" smd rect (at 0 0 180) (size 1 1.5) (layers "F.Cu" "F.Mask") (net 45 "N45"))
  (pad "3" smd custom (at 1.3 0 180) (size 1 0.5) (layers "F.Cu" "F.Mask") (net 5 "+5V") (zone_connect 2) (thermal_bridge_angle 45)
   (options (clearance outline) (anchor rect)) (primitives)))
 (gr_rect (start 111 49) (end 183.5 139.5) (stroke (width 0.05) (type default)) (fill none) (layer "Edge.Cuts"))
 (segment (start 171.195 87.99) (end 170.3 88.885) (width 0.2) (layer "F.Cu") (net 2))
 (segment (start 170.3 88.885) (end 170.3 89.835) (width 0.2) (layer "F.Cu") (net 2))
 (segment (start 175 87.99) (end 171.195 87.99) (width 0.2) (layer "F.Cu") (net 2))
 (segment (start 170.85 87.5) (end 170.3 86.95) (width 0.2) (layer "F.Cu") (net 45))
 (segment (start 170.3 86.95) (end 170.3 86) (width 0.2) (layer "F.Cu") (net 45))
 (segment (start 172.95 87.5) (end 170.85 87.5) (width 0.2) (layer "F.Cu") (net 45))
 (segment (start 175 85.45) (end 172.95 87.5) (width 0.2) (layer "F.Cu") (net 45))
 (segment (start 175 82.91) (end 174.15 83.76) (width 0.2) (layer "F.Cu") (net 37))
 (segment (start 170.3 83.115) (end 170.3 82.165) (width 0.2) (layer "F.Cu") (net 37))
 (segment (start 170.945 83.76) (end 170.3 83.115) (width 0.2) (layer "F.Cu") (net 37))
 (segment (start 174.15 83.76) (end 170.945 83.76) (width 0.2) (layer "F.Cu") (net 37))
 (segment (start 170.3 79.28) (end 170.3 78.33) (width 0.2) (layer "F.Cu") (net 6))
 (segment (start 175 80.37) (end 171.39 80.37) (width 0.2) (layer "F.Cu") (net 6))
 (segment (start 171.39 80.37) (end 170.3 79.28) (width 0.2) (layer "F.Cu") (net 6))
 (segment (start 119.5 135.5) (end 114 130) (width 0.2) (layer "B.Cu") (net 41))
 (segment (start 162.35 131.37) (end 158.22 135.5) (width 0.2) (layer "B.Cu") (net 41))
 (segment (start 158.22 135.5) (end 119.5 135.5) (width 0.2) (layer "B.Cu") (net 41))
 (segment (start 114 91.915) (end 122 83.915) (width 0.2) (layer "B.Cu") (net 41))
 (segment (start 114 130) (end 114 91.915) (width 0.2) (layer "B.Cu") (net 41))
 (segment (start 125.5 84) (end 126.2 83.3) (width 0.2) (layer "F.Cu") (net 40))
 (segment (start 125 84) (end 125.5 84) (width 0.2) (layer "F.Cu") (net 40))
 (segment (start 126.2 83.3) (end 126.2 82.165) (width 0.2) (layer "F.Cu") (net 40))
 (via (at 125 84) (size 0.6) (drill 0.3) (layers "F.Cu" "B.Cu") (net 40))
 (segment (start 124.625 84) (end 125 84) (width 0.2) (layer "B.Cu") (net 40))
 (segment (start 122 81.375) (end 124.625 84) (width 0.2) (layer "B.Cu") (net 40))
 (segment (start 126 86.2) (end 126.2 86) (width 0.2) (layer "F.Cu") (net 42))
 (segment (start 126 87.35) (end 126 86.2) (width 0.2) (layer "F.Cu") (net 42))
 (via (at 126 87.35) (size 0.6) (drill 0.3) (layers "F.Cu" "B.Cu") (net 42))
 (segment (start 122 86.455) (end 125.105 86.455) (width 0.2) (layer "B.Cu") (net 42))
 (segment (start 125.105 86.455) (end 126 87.35) (width 0.2) (layer "B.Cu") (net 42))
 (segment (start 126.2 90.785) (end 126.2 89.835) (width 0.2) (layer "F.Cu") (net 4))
 (segment (start 127.5 91.5) (end 126.915 91.5) (width 0.2) (layer "F.Cu") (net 4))
 (segment (start 123.5 90.495) (end 123.5 91.5) (width 0.2) (layer "F.Cu") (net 4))
 (segment (start 126.915 91.5) (end 126.2 90.785) (width 0.2) (layer "F.Cu") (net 4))
 (segment (start 122 88.995) (end 123.5 90.495) (width 0.2) (layer "F.Cu") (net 4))
 (via (at 123.5 91.5) (size 0.6) (drill 0.3) (layers "F.Cu" "B.Cu") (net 4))
 (via (at 127.5 91.5) (size 0.6) (drill 0.3) (layers "F.Cu" "B.Cu") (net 4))
 (segment (start 123.5 91.5) (end 127.5 91.5) (width 0.2) (layer "B.Cu") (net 4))
 (segment (start 126.045 77.225) (end 126.2 77.38) (width 0.2) (layer "F.Cu") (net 39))
 (segment (start 126.2 77.38) (end 126.2 78.33) (width 0.2) (layer "F.Cu") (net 39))
 (segment (start 123.61 77.225) (end 126.045 77.225) (width 0.2) (layer "F.Cu") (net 39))
 (segment (start 122 78.835) (end 123.61 77.225) (width 0.2) (layer "F.Cu") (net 39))
 (segment (start 120.5 78.035) (end 120.5 92) (width 0.2) (layer "F.Cu") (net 3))
 (segment (start 120.5 92) (end 121 92.5) (width 0.2) (layer "F.Cu") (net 3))
 (segment (start 156 100) (end 163 100) (width 0.2) (layer "F.Cu") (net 3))
 (segment (start 171 92) (end 169 94) (width 0.2) (layer "F.Cu") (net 3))
 (segment (start 124.9 90.59) (end 129.77 95.46) (width 0.2) (layer "F.Cu") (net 3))
 (segment (start 124 92.5) (end 124.9 91.6) (width 0.2) (layer "F.Cu") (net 3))
 (segment (start 125.925 76) (end 122.535 76) (width 0.2) (layer "F.Cu") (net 3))
 (segment (start 124.9 89.835) (end 124.9 90.59) (width 0.2) (layer "F.Cu") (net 3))
 (segment (start 176 92) (end 171 92) (width 0.2) (layer "F.Cu") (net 3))
 (segment (start 122.535 76) (end 120.5 78.035) (width 0.2) (layer "F.Cu") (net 3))
 (segment (start 127.5 78.33) (end 127.5 77.575) (width 0.2) (layer "F.Cu") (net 3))
 (segment (start 169 94) (end 169 89.835) (width 0.2) (layer "F.Cu") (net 3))
 (segment (start 137.14 95.46) (end 151.46 95.46) (width 0.2) (layer "F.Cu") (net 3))
 (segment (start 124.9 91.6) (end 124.9 89.835) (width 0.2) (layer "F.Cu") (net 3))
 (segment (start 177.5 80) (end 177.5 90.5) (width 0.2) (layer "F.Cu") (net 3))
 (segment (start 129.77 95.46) (end 137.14 95.46) (width 0.2) (layer "F.Cu") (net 3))
 (segment (start 163 100) (end 169 94) (width 0.2) (layer "F.Cu") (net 3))
 (segment (start 127.5 77.575) (end 125.925 76) (width 0.2) (layer "F.Cu") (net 3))
 (segment (start 175.83 78.33) (end 177.5 80) (width 0.2) (layer "F.Cu") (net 3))
 (segment (start 171.6 78.33) (end 175.83 78.33) (width 0.2) (layer "F.Cu") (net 3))
 (segment (start 177.5 90.5) (end 176 92) (width 0.2) (layer "F.Cu") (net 3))
 (segment (start 121 92.5) (end 124 92.5) (width 0.2) (layer "F.Cu") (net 3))
 (segment (start 151.46 95.46) (end 156 100) (width 0.2) (layer "F.Cu") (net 3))
 (segment (start 133.54 95.46) (end 137.14 95.46) (width 0.2) (layer "B.Cu") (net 3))
 (segment (start 136.95 131.37) (end 133 127.42) (width 0.2) (layer "B.Cu") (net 3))
 (segment (start 133 96) (end 133.54 95.46) (width 0.2) (layer "B.Cu") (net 3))
 (segment (start 133 127.42) (end 133 96) (width 0.2) (layer "B.Cu") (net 3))
 (segment (start 173 90) (end 171.765 90) (width 0.2) (layer "F.Cu") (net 1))
 (segment (start 171.765 90) (end 171.6 89.835) (width 0.2) (layer "F.Cu") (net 1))
 (segment (start 169 78.33) (end 169 80) (width 0.2) (layer "F.Cu") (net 1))
 (via (at 169 80) (size 0.6) (drill 0.3) (layers "F.Cu" "B.Cu") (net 1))
 (via (at 173 90) (size 0.6) (drill 0.3) (layers "F.Cu" "B.Cu") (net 1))
 (segment (start 173 84) (end 173 90) (width 0.2) (layer "B.Cu") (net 1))
 (segment (start 169 80) (end 173 84) (width 0.2) (layer "B.Cu") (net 1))
 (segment (start 154.73 131.37) (end 154.73 125.77) (width 0.2) (layer "B.Cu") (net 1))
 (segment (start 167.978393 112.521607) (end 167.978393 81.021607) (width 0.2) (layer "B.Cu") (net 1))
 (segment (start 167.978393 81.021607) (end 169 80) (width 0.2) (layer "B.Cu") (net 1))
 (segment (start 154.73 125.77) (end 167.978393 112.521607) (width 0.2) (layer "B.Cu") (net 1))
 (segment (start 171.6 86) (end 171.6 85.245) (width 0.2) (layer "F.Cu") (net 38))
 (segment (start 169 84) (end 169 82.165) (width 0.2) (layer "F.Cu") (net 38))
 (segment (start 169 82.645) (end 169 82.165) (width 0.2) (layer "F.Cu") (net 38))
 (segment (start 171.6 85.245) (end 169 82.645) (width 0.2) (layer "F.Cu") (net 38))
 (via (at 169 84) (size 0.6) (drill 0.3) (layers "F.Cu" "B.Cu") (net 38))
 (segment (start 157.45 131.37) (end 169 119.82) (width 0.2) (layer "B.Cu") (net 38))
 (segment (start 157.27 131.37) (end 157.45 131.37) (width 0.2) (layer "B.Cu") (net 38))
 (segment (start 169 119.82) (end 169 84) (width 0.2) (layer "B.Cu") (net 38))
 (segment (start 124.5 88) (end 124 87.5) (width 0.2) (layer "F.Cu") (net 5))
 (segment (start 127.5 89.835) (end 127.5 89.08) (width 0.2) (layer "F.Cu") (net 5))
 (segment (start 167.5 81.5) (end 168 81) (width 0.2) (layer "F.Cu") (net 5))
 (segment (start 127.5 89.835) (end 130.585 92.92) (width 0.2) (layer "F.Cu") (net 5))
 (segment (start 169 86) (end 167.5 84.5) (width 0.2) (layer "F.Cu") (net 5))
 (segment (start 126.42 88) (end 124.5 88) (width 0.2) (layer "F.Cu") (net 5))
 (segment (start 171.19 81) (end 171.6 81.41) (width 0.2) (layer "F.Cu") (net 5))
 (segment (start 124 79.23) (end 124.9 78.33) (width 0.2) (layer "F.Cu") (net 5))
 (segment (start 127.5 89.08) (end 126.42 88) (width 0.2) (layer "F.Cu") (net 5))
 (segment (start 167.5 84.5) (end 167.5 81.5) (width 0.2) (layer "F.Cu") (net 5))
 (segment (start 171.6 81.41) (end 171.6 82.165) (width 0.2) (layer "F.Cu") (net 5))
 (segment (start 124 87.5) (end 124 79.23) (width 0.2) (layer "F.Cu") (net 5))
 (segment (start 168 81) (end 171.19 81) (width 0.2) (layer "F.Cu") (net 5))
 (segment (start 130.585 92.92) (end 137.14 92.92) (width 0.2) (layer "F.Cu") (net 5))
 (segment (start 167 88) (end 169 86) (width 0.2) (layer "F.Cu") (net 5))
 (via (at 167 88) (size 0.6) (drill 0.3) (layers "F.Cu" "B.Cu") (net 5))
 (segment (start 132 95.5) (end 134.58 92.92) (width 0.2) (layer "B.Cu") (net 5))
 (segment (start 163 100) (end 167 96) (width 0.2) (layer "B.Cu") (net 5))
 (segment (start 148.92 92.92) (end 156 100) (width 0.2) (layer "B.Cu") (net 5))
 (segment (start 167 96) (end 167 88) (width 0.2) (layer "B.Cu") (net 5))
 (segment (start 134.41 131.37) (end 132.37 131.37) (width 0.2) (layer "B.Cu") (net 5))
 (segment (start 134.58 92.92) (end 137.14 92.92) (width 0.2) (layer "B.Cu") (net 5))
 (segment (start 156 100) (end 163 100) (width 0.2) (layer "B.Cu") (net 5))
 (segment (start 132 131) (end 132 95.5) (width 0.2) (layer "B.Cu") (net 5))
 (segment (start 137.14 92.92) (end 148.92 92.92) (width 0.2) (layer "B.Cu") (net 5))
 (segment (start 132.37 131.37) (end 132 131) (width 0.2) (layer "B.Cu") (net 5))
 (segment (start 128.057219 80.5) (end 129 81.442781) (width 0.2) (layer "F.Cu") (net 46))
 (segment (start 129 84.5) (end 127.5 86) (width 0.2) (layer "F.Cu") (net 46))
 (segment (start 129 81.442781) (end 129 84.5) (width 0.2) (layer "F.Cu") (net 46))
 (segment (start 124.9 82.165) (end 124.9 81.41) (width 0.2) (layer "F.Cu") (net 46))
 (segment (start 124.9 81.41) (end 125.81 80.5) (width 0.2) (layer "F.Cu") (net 46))
 (segment (start 125.81 80.5) (end 128.057219 80.5) (width 0.2) (layer "F.Cu") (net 46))
 (segment (start 124.9 85.245) (end 125.645 84.5) (width 0.2) (layer "F.Cu") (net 44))
 (segment (start 124.9 86) (end 124.9 85.245) (width 0.2) (layer "F.Cu") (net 44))
 (segment (start 127.5 84) (end 127.5 82.165) (width 0.2) (layer "F.Cu") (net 44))
 (segment (start 127 84.5) (end 127.5 84) (width 0.2) (layer "F.Cu") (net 44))
 (segment (start 125.645 84.5) (end 127 84.5) (width 0.2) (layer "F.Cu") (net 44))
 (via (at 127.5 84) (size 0.6) (drill 0.3) (layers "F.Cu" "B.Cu") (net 44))
 (segment (start 159.81 131.37) (end 159.81 132.69) (width 0.2) (layer "B.Cu") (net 44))
 (segment (start 158.5 134) (end 120 134) (width 0.2) (layer "B.Cu") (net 44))
 (segment (start 115 129) (end 115 98.5) (width 0.2) (layer "B.Cu") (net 44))
 (segment (start 120 134) (end 115 129) (width 0.2) (layer "B.Cu") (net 44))
 (segment (start 126.269239 88) (end 127.5 86.769239) (width 0.2) (layer "B.Cu") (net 44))
 (segment (start 125.5 88) (end 126.269239 88) (width 0.2) (layer "B.Cu") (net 44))
 (segment (start 115 98.5) (end 125.5 88) (width 0.2) (layer "B.Cu") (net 44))
 (segment (start 127.5 86.769239) (end 127.5 84) (width 0.2) (layer "B.Cu") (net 44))
 (segment (start 159.81 132.69) (end 158.5 134) (width 0.2) (layer "B.Cu") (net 44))
 (segment (start 148.44 62.44) (end 140 54) (width 0.2) (layer "F.Cu") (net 22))
 (segment (start 114 61) (end 114 129.5) (width 0.2) (layer "F.Cu") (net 22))
 (segment (start 139 135.5) (end 142.03 132.47) (width 0.2) (layer "F.Cu") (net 22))
 (segment (start 160 62.44) (end 148.44 62.44) (width 0.2) (layer "F.Cu") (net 22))
 (segment (start 120 135.5) (end 139 135.5) (width 0.2) (layer "F.Cu") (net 22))
 (segment (start 140 54) (end 121 54) (width 0.2) (layer "F.Cu") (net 22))
 (segment (start 114 129.5) (end 120 135.5) (width 0.2) (layer "F.Cu") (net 22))
 (segment (start 121 54) (end 114 61) (width 0.2) (layer "F.Cu") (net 22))
 (segment (start 142.03 132.47) (end 142.03 131.37) (width 0.2) (layer "F.Cu") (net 22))
 (segment (start 148.52 64.98) (end 160 64.98) (width 0.2) (layer "F.Cu") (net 23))
 (segment (start 148.5 65) (end 148.52 64.98) (width 0.2) (layer "F.Cu") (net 23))
 (segment (start 115 62) (end 121.5 55.5) (width 0.2) (layer "F.Cu") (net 23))
 (segment (start 139.49 131.37) (end 139.49 133.01) (width 0.2) (layer "F.Cu") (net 23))
 (segment (start 120.5 134.5) (end 115 129) (width 0.2) (layer "F.Cu") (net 23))
 (segment (start 138 134.5) (end 120.5 134.5) (width 0.2) (layer "F.Cu") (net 23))
 (segment (start 139.49 133.01) (end 138 134.5) (width 0.2) (layer "F.Cu") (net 23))
 (segment (start 121.5 55.5) (end 139 55.5) (width 0.2) (layer "F.Cu") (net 23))
 (segment (start 139 55.5) (end 148.5 65) (width 0.2) (layer "F.Cu") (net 23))
 (segment (start 115 129) (end 115 62) (width 0.2) (layer "F.Cu") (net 23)))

